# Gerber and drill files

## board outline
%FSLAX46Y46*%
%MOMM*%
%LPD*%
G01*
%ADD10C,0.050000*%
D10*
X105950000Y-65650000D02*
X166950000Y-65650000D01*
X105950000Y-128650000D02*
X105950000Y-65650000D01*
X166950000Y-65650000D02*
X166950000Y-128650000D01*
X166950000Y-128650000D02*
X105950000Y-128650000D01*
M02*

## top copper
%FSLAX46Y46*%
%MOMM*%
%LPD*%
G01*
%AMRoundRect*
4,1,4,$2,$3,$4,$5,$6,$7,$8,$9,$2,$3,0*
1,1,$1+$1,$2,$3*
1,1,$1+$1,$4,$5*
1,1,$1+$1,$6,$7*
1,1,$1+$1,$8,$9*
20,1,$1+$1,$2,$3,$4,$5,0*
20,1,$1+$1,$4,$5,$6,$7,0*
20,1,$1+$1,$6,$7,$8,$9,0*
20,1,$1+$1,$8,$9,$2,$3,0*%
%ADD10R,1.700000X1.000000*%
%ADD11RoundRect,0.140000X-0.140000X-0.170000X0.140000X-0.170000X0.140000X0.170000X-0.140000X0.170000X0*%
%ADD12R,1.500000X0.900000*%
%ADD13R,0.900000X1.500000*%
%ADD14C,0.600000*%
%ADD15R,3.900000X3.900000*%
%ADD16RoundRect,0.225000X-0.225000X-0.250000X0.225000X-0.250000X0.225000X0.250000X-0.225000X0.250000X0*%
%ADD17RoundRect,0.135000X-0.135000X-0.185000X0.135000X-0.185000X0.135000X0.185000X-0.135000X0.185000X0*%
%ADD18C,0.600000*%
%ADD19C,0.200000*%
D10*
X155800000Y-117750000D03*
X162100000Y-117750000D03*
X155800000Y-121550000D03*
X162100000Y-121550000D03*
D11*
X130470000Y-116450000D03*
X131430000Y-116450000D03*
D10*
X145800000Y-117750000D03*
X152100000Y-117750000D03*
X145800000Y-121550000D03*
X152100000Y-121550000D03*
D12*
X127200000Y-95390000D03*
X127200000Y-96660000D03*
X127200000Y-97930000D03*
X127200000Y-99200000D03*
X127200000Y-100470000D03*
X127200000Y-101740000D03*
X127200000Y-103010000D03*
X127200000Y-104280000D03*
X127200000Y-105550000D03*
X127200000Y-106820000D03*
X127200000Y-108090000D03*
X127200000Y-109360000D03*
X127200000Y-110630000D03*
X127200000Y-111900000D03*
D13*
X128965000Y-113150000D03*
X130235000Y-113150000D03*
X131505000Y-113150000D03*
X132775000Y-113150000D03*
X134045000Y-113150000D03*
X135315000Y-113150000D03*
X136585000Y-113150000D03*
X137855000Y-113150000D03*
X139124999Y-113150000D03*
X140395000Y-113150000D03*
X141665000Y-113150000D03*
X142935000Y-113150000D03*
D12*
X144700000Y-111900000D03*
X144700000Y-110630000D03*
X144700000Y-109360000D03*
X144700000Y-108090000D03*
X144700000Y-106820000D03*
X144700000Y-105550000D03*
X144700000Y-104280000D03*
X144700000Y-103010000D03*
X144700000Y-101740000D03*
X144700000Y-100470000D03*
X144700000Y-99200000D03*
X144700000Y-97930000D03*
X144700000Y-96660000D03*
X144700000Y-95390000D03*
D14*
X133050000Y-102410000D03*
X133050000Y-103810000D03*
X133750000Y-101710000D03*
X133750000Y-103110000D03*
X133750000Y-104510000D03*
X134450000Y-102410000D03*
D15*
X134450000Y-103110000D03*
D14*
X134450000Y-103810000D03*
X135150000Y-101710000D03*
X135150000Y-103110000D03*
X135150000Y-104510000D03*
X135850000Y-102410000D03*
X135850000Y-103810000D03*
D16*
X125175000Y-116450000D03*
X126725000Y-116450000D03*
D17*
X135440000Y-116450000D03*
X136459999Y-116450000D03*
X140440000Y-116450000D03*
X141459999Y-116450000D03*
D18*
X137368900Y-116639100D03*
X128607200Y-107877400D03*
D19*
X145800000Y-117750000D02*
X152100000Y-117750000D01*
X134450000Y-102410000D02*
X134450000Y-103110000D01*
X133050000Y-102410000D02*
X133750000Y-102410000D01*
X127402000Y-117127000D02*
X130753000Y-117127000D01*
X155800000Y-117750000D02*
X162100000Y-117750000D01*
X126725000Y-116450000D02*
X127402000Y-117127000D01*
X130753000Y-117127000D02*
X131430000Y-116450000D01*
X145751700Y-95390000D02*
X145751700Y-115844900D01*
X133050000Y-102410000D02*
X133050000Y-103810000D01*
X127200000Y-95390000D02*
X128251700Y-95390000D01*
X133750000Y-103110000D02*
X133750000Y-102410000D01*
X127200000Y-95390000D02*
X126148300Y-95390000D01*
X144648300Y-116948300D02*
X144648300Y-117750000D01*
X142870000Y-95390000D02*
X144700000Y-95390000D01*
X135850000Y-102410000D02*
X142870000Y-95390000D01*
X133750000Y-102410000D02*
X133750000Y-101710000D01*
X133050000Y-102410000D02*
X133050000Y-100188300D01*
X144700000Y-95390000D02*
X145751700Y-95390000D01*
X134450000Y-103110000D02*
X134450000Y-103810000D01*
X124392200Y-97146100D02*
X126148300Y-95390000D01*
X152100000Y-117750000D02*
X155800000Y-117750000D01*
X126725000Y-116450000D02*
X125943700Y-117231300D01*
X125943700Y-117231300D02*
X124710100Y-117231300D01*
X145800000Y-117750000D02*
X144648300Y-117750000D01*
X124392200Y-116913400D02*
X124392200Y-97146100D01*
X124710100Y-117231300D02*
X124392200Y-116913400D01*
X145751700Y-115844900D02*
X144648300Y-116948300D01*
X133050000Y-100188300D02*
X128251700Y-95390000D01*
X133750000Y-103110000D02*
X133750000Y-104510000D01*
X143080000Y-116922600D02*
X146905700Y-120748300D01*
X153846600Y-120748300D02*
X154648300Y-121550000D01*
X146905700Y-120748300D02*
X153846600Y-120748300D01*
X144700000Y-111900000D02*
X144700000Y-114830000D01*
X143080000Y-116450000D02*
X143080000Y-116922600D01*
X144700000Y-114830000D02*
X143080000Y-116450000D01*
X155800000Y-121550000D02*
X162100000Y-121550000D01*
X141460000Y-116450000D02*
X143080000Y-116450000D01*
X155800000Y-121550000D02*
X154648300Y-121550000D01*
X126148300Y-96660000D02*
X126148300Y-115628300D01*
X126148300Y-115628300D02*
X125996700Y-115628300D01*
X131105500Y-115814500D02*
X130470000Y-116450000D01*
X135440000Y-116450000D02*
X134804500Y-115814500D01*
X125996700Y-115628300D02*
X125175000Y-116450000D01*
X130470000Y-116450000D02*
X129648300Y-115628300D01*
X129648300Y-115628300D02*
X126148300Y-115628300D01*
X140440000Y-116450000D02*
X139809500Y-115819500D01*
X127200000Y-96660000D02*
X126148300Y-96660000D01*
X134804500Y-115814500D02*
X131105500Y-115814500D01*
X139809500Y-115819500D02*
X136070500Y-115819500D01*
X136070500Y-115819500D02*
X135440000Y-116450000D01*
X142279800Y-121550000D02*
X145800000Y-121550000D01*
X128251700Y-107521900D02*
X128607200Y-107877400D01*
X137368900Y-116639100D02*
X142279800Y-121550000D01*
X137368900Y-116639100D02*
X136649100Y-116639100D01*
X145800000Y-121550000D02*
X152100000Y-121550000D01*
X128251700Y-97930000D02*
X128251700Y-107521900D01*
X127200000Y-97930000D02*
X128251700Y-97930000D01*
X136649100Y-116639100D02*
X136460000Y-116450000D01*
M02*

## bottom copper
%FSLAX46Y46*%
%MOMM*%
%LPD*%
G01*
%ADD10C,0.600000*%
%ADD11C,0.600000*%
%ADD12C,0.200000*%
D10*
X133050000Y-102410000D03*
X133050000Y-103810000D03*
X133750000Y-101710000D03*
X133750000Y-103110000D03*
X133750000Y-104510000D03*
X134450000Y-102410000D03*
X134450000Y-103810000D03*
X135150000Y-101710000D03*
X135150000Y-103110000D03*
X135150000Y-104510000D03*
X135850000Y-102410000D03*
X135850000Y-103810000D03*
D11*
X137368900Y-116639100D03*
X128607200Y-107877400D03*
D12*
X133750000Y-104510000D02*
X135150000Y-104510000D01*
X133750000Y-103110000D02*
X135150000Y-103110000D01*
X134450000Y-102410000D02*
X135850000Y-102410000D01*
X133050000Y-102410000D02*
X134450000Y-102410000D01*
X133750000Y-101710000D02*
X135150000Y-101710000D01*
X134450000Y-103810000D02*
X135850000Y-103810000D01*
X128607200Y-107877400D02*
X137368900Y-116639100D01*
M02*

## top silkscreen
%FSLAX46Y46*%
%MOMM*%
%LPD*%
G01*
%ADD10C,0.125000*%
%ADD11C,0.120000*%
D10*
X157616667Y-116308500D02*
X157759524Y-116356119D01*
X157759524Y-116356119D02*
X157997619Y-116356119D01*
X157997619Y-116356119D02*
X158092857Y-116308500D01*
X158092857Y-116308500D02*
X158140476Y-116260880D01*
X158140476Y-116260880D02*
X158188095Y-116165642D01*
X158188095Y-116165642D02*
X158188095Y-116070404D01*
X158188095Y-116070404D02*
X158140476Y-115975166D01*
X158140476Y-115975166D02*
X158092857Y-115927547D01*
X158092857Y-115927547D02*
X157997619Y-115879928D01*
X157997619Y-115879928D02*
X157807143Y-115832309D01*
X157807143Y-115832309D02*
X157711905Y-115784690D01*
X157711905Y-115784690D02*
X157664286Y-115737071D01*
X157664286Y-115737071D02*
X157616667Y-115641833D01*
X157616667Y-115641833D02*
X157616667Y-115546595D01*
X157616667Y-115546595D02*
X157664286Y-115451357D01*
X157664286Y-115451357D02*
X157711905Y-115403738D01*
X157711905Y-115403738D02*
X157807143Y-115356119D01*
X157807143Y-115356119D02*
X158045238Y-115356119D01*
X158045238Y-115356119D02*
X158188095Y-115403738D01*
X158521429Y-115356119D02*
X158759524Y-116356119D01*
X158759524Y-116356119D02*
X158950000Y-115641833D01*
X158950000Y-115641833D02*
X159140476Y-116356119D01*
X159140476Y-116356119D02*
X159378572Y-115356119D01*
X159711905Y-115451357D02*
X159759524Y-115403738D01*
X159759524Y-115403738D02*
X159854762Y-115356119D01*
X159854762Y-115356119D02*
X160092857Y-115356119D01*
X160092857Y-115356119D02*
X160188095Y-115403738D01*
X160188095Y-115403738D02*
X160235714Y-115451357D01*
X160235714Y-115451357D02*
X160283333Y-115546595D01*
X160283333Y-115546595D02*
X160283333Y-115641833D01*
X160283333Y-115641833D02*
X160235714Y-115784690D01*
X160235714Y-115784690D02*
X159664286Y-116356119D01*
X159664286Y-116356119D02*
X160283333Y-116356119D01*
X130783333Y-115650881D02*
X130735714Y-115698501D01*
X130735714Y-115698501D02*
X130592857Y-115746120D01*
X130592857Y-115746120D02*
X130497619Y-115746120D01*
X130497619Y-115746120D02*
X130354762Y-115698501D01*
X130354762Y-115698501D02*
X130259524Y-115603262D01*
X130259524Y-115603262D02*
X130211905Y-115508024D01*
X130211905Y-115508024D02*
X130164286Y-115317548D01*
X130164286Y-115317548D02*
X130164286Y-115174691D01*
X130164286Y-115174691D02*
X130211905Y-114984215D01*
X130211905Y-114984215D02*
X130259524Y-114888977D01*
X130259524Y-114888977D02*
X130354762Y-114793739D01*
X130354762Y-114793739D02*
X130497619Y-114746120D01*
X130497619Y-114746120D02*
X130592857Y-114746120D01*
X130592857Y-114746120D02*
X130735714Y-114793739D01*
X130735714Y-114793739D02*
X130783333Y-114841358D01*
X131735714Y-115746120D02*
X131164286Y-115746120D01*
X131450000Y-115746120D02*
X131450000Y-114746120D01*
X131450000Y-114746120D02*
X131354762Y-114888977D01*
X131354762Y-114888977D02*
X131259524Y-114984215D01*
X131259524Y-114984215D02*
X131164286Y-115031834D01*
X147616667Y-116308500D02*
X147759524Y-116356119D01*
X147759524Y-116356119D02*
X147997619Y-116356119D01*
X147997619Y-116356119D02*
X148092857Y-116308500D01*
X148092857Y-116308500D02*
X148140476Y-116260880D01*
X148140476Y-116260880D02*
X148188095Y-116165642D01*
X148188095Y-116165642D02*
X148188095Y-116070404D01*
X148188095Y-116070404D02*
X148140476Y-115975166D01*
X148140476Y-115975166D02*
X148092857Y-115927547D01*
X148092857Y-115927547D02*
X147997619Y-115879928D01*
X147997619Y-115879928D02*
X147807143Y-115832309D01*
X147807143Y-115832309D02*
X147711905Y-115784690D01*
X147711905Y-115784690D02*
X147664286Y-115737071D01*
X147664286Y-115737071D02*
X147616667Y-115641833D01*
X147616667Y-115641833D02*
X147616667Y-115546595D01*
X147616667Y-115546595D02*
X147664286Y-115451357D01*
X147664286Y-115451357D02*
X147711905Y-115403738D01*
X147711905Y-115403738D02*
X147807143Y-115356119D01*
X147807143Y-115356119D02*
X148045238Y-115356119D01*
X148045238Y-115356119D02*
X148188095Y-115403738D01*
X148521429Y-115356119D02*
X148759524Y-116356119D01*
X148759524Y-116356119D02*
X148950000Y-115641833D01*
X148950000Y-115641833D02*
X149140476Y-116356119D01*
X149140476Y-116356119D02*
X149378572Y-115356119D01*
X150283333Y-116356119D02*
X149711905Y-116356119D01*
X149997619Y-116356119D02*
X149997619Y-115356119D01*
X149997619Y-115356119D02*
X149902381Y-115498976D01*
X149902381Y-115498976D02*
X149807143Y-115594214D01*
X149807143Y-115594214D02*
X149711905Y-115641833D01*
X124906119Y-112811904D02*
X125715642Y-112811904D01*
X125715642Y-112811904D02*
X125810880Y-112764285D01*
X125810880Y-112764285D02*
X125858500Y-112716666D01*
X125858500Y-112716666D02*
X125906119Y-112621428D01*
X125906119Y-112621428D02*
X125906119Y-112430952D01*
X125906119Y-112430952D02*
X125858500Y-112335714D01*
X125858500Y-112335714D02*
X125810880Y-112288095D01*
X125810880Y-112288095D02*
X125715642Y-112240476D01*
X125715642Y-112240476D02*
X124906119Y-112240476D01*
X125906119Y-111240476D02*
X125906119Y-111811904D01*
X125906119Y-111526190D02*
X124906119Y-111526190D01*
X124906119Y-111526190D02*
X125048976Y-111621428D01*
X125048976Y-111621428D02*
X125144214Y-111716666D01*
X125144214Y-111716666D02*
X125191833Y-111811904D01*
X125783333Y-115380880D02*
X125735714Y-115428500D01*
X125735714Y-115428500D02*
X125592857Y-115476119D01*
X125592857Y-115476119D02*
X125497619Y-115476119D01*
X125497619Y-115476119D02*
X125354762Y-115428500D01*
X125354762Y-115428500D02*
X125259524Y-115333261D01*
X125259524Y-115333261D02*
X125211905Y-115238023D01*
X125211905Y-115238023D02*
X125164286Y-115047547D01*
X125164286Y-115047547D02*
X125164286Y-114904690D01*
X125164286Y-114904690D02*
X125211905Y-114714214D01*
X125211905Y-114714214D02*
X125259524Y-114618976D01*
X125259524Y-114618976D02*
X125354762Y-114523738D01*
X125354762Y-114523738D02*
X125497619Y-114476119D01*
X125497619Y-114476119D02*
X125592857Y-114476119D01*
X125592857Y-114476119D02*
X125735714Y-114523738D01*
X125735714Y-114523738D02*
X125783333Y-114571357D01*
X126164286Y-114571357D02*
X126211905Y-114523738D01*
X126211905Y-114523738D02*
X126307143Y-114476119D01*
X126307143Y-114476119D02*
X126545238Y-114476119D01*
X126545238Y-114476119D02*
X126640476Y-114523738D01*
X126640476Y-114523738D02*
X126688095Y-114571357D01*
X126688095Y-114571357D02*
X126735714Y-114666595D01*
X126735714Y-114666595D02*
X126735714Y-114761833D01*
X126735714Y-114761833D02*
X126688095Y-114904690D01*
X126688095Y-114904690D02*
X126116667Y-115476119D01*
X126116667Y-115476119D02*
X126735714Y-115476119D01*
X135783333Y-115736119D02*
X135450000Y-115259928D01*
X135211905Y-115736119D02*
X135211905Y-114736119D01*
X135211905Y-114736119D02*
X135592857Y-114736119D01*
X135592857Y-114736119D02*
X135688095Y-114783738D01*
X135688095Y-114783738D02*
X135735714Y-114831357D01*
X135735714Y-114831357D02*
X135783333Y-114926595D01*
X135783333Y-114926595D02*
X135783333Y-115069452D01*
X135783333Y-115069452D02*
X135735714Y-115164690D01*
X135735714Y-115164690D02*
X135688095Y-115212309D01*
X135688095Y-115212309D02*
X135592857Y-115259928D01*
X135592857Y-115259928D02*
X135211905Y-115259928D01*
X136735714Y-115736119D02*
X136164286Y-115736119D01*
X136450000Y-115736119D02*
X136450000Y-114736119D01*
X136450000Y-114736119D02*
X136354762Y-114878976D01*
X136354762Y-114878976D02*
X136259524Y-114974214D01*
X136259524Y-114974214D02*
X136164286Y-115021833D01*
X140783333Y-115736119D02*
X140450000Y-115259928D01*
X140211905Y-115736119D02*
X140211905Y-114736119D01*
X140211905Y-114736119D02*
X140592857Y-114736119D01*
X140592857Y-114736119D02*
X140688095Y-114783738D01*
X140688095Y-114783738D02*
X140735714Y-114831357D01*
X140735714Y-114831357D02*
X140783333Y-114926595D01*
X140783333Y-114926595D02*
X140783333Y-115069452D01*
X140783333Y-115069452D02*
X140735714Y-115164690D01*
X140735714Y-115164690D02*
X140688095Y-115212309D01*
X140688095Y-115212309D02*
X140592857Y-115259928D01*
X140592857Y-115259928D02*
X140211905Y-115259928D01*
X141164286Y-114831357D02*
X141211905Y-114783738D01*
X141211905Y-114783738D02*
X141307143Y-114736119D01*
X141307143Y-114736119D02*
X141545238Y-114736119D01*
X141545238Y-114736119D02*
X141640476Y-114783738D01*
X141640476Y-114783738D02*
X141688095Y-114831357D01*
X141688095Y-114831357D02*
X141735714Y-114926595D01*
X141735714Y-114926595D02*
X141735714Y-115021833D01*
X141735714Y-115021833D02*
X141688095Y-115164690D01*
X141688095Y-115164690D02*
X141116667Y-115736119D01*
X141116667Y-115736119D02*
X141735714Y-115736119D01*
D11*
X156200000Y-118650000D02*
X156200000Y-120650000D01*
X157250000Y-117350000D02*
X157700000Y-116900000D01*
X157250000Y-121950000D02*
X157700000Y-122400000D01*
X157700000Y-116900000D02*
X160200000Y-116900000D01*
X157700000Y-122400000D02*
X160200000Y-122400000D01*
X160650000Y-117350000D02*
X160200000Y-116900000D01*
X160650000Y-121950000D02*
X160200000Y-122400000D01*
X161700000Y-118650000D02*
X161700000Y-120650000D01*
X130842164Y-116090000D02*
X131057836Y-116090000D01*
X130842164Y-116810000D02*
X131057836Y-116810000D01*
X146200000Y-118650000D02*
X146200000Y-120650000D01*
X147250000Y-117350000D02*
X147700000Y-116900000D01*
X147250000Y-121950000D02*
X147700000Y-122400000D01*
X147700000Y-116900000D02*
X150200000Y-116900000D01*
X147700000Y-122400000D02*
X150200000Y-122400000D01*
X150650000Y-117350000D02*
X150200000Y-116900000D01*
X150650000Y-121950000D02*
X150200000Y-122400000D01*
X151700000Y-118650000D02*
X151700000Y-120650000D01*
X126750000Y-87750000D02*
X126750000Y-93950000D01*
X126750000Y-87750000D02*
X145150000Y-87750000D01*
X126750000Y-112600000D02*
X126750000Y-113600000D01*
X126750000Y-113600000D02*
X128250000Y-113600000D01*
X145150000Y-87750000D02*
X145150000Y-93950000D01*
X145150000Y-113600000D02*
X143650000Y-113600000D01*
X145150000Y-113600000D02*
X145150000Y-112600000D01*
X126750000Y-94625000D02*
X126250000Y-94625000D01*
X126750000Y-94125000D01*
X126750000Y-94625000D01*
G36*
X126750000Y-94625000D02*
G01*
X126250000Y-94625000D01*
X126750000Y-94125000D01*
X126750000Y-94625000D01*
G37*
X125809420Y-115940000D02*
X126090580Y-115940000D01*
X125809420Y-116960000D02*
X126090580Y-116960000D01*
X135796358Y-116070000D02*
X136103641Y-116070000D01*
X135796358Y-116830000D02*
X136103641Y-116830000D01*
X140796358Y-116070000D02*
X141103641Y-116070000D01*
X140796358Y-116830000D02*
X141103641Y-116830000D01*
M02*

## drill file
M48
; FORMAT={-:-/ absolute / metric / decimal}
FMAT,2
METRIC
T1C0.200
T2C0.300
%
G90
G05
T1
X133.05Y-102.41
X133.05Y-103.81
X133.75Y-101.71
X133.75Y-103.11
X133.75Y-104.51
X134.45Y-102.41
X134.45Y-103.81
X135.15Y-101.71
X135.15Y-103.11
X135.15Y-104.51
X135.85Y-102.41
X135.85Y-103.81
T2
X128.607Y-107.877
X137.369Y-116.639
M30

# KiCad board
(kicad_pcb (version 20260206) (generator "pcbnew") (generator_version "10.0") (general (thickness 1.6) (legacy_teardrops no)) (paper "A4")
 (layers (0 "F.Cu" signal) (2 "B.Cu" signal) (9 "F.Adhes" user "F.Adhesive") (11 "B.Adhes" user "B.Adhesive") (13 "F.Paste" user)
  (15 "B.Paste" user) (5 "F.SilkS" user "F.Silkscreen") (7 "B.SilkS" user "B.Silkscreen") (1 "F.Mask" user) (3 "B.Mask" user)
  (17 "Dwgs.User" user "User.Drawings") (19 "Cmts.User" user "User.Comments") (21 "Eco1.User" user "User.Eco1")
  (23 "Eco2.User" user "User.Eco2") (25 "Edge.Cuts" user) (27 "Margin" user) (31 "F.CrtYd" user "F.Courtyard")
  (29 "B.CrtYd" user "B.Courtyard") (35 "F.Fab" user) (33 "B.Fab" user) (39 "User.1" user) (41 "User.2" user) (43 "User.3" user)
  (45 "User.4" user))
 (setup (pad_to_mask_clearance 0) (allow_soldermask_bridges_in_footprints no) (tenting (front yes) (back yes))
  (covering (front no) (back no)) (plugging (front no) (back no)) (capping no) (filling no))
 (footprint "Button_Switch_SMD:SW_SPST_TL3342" (layer "F.Cu") (at 158.95 119.65)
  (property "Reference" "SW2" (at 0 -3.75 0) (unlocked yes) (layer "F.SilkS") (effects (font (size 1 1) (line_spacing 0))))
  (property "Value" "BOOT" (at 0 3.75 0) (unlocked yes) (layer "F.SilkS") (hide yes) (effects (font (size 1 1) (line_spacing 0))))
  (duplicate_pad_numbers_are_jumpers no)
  (fp_line (start -2.75 -1) (end -2.75 1) (stroke (width 0.12) (type solid)) (layer "F.SilkS"))
  (fp_line (start -1.7 -2.3) (end -1.25 -2.75) (stroke (width 0.12) (type solid)) (layer "F.SilkS"))
  (fp_line (start -1.7 2.3) (end -1.25 2.75) (stroke (width 0.12) (type solid)) (layer "F.SilkS"))
  (fp_line (start -1.25 -2.75) (end 1.25 -2.75) (stroke (width 0.12) (type solid)) (layer "F.SilkS"))
  (fp_line (start -1.25 2.75) (end 1.25 2.75) (stroke (width 0.12) (type solid)) (layer "F.SilkS"))
  (fp_line (start 1.7 -2.3) (end 1.25 -2.75) (stroke (width 0.12) (type solid)) (layer "F.SilkS"))
  (fp_line (start 1.7 2.3) (end 1.25 2.75) (stroke (width 0.12) (type solid)) (layer "F.SilkS"))
  (fp_line (start 2.75 -1) (end 2.75 1) (stroke (width 0.12) (type solid)) (layer "F.SilkS"))
  (pad "1" smd rect (at -3.15 -1.9) (size 1.7 1) (layers "F.Cu" "F.Mask" "F.Paste") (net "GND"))
  (pad "1" smd rect (at 3.15 -1.9) (size 1.7 1) (layers "F.Cu" "F.Mask" "F.Paste") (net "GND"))
  (pad "2" smd rect (at -3.15 1.9) (size 1.7 1) (layers "F.Cu" "F.Mask" "F.Paste") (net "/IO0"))
  (pad "2" smd rect (at 3.15 1.9) (size 1.7 1) (layers "F.Cu" "F.Mask" "F.Paste") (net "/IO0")))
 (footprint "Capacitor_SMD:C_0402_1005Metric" (layer "F.Cu") (at 130.95 116.45)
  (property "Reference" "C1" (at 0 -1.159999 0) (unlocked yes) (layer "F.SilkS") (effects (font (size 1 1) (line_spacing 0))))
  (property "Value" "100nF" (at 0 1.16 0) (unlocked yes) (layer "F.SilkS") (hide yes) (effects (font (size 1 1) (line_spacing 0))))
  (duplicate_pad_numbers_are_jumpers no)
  (fp_line (start -0.107836 -0.36) (end 0.107836 -0.36) (stroke (width 0.12) (type solid)) (layer "F.SilkS"))
  (fp_line (start -0.107836 0.36) (end 0.107836 0.36) (stroke (width 0.12) (type solid)) (layer "F.SilkS"))
  (pad "1" smd roundrect (at -0.48 0) (size 0.56 0.62) (layers "F.Cu" "F.Mask" "F.Paste") (roundrect_rratio 0.25) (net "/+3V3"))
  (pad "2" smd roundrect (at 0.48 0) (size 0.56 0.62) (layers "F.Cu" "F.Mask" "F.Paste") (roundrect_rratio 0.25) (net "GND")))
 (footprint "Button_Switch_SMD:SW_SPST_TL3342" (layer "F.Cu") (at 148.95 119.65)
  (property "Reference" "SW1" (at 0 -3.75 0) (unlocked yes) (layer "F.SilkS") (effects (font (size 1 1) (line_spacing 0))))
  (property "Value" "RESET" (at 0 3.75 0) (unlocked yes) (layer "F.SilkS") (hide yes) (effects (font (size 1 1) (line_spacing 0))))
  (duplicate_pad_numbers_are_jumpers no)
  (fp_line (start -2.75 -1) (end -2.75 1) (stroke (width 0.12) (type solid)) (layer "F.SilkS"))
  (fp_line (start -1.7 -2.3) (end -1.25 -2.75) (stroke (width 0.12) (type solid)) (layer "F.SilkS"))
  (fp_line (start -1.7 2.3) (end -1.25 2.75) (stroke (width 0.12) (type solid)) (layer "F.SilkS"))
  (fp_line (start -1.25 -2.75) (end 1.25 -2.75) (stroke (width 0.12) (type solid)) (layer "F.SilkS"))
  (fp_line (start -1.25 2.75) (end 1.25 2.75) (stroke (width 0.12) (type solid)) (layer "F.SilkS"))
  (fp_line (start 1.7 -2.3) (end 1.25 -2.75) (stroke (width 0.12) (type solid)) (layer "F.SilkS"))
  (fp_line (start 1.7 2.3) (end 1.25 2.75) (stroke (width 0.12) (type solid)) (layer "F.SilkS"))
  (fp_line (start 2.75 -1) (end 2.75 1) (stroke (width 0.12) (type solid)) (layer "F.SilkS"))
  (pad "1" smd rect (at -3.15 -1.9) (size 1.7 1) (layers "F.Cu" "F.Mask" "F.Paste") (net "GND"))
  (pad "1" smd rect (at 3.15 -1.9) (size 1.7 1) (layers "F.Cu" "F.Mask" "F.Paste") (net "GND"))
  (pad "2" smd rect (at -3.15 1.9) (size 1.7 1) (layers "F.Cu" "F.Mask" "F.Paste") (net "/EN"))
  (pad "2" smd rect (at 3.15 1.9) (size 1.7 1) (layers "F.Cu" "F.Mask" "F.Paste") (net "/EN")))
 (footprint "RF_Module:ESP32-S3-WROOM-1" (layer "F.Cu") (at 135.95 100.65)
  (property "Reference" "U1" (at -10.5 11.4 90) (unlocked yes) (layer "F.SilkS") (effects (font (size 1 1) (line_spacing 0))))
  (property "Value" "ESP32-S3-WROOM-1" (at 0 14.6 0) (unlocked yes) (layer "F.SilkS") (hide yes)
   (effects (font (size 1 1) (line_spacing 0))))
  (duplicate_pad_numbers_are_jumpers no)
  (fp_line (start -9.2 -12.9) (end -9.2 -6.7) (stroke (width 0.12) (type solid)) (layer "F.SilkS"))
  (fp_line (start -9.2 -12.9) (end 9.2 -12.9) (stroke (width 0.12) (type solid)) (layer "F.SilkS"))
  (fp_line (start -9.2 11.95) (end -9.2 12.95) (stroke (width 0.12) (type solid)) (layer "F.SilkS"))
  (fp_line (start -9.2 12.95) (end -7.7 12.95) (stroke (width 0.12) (type solid)) (layer "F.SilkS"))
  (fp_line (start 9.2 -12.9) (end 9.2 -6.7) (stroke (width 0.12) (type solid)) (layer "F.SilkS"))
  (fp_line (start 9.2 12.95) (end 7.7 12.95) (stroke (width 0.12) (type solid)) (layer "F.SilkS"))
  (fp_line (start 9.2 12.95) (end 9.2 11.95) (stroke (width 0.12) (type solid)) (layer "F.SilkS"))
  (fp_poly
   (pts (xy -9.2 -6.025) (xy -9.7 -6.025) (xy -9.2 -6.525) (xy -9.2 -6.025)) (stroke (width 0.12) (type solid)) (fill yes) (layer "F.SilkS"))
  (pad "" smd rect (at -2.9 1.06) (size 0.9 0.9) (layers "F.Paste"))
  (pad "" smd rect (at -2.9 2.46 270) (size 0.9 0.9) (layers "F.Paste"))
  (pad "" smd rect (at -2.9 3.86) (size 0.9 0.9) (layers "F.Paste"))
  (pad "" smd rect (at -1.5 1.06 270) (size 0.9 0.9) (layers "F.Paste"))
  (pad "" smd rect (at -1.5 2.46 270) (size 0.9 0.9) (layers "F.Paste"))
  (pad "" smd rect (at -1.5 3.86 270) (size 0.9 0.9) (layers "F.Paste"))
  (pad "" smd rect (at -0.1 1.06 270) (size 0.9 0.9) (layers "F.Paste"))
  (pad "" smd rect (at -0.1 2.46 270) (size 0.9 0.9) (layers "F.Paste"))
  (pad "" smd rect (at -0.1 3.86 270) (size 0.9 0.9) (layers "F.Paste"))
  (pad "1" smd rect (at -8.75 -5.26) (size 1.5 0.9) (layers "F.Cu" "F.Mask" "F.Paste") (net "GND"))
  (pad "2" smd rect (at -8.75 -3.99) (size 1.5 0.9) (layers "F.Cu" "F.Mask" "F.Paste") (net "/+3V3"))
  (pad "3" smd rect (at -8.75 -2.72) (size 1.5 0.9) (layers "F.Cu" "F.Mask" "F.Paste") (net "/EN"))
  (pad "4" smd rect (at -8.75 -1.45) (size 1.5 0.9) (layers "F.Cu" "F.Mask" "F.Paste") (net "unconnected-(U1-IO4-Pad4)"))
  (pad "5" smd rect (at -8.75 -0.18) (size 1.5 0.9) (layers "F.Cu" "F.Mask" "F.Paste") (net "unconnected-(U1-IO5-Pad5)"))
  (pad "6" smd rect (at -8.75 1.09) (size 1.5 0.9) (layers "F.Cu" "F.Mask" "F.Paste") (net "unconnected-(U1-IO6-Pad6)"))
  (pad "7" smd rect (at -8.75 2.36) (size 1.5 0.9) (layers "F.Cu" "F.Mask" "F.Paste") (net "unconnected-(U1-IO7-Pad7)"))
  (pad "8" smd rect (at -8.75 3.63) (size 1.5 0.9) (layers "F.Cu" "F.Mask" "F.Paste") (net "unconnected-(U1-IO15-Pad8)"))
  (pad "9" smd rect (at -8.75 4.9) (size 1.5 0.9) (layers "F.Cu" "F.Mask" "F.Paste") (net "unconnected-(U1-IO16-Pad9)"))
  (pad "10" smd rect (at -8.75 6.17) (size 1.5 0.9) (layers "F.Cu" "F.Mask" "F.Paste") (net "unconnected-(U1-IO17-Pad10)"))
  (pad "11" smd rect (at -8.75 7.44) (size 1.5 0.9) (layers "F.Cu" "F.Mask" "F.Paste") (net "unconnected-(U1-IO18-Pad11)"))
  (pad "12" smd rect (at -8.75 8.71) (size 1.5 0.9) (layers "F.Cu" "F.Mask" "F.Paste") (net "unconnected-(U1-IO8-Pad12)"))
  (pad "13" smd rect (at -8.75 9.98) (size 1.5 0.9) (layers "F.Cu" "F.Mask" "F.Paste") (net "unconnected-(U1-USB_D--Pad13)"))
  (pad "14" smd rect (at -8.75 11.25 180) (size 1.5 0.9) (layers "F.Cu" "F.Mask" "F.Paste") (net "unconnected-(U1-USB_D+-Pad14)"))
  (pad "15" smd rect (at -6.985 12.5 270) (size 1.5 0.9) (layers "F.Cu" "F.Mask" "F.Paste") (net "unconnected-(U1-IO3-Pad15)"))
  (pad "16" smd rect (at -5.715 12.5 270) (size 1.5 0.9) (layers "F.Cu" "F.Mask" "F.Paste") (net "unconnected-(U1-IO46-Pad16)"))
  (pad "17" smd rect (at -4.445 12.5 270) (size 1.5 0.9) (layers "F.Cu" "F.Mask" "F.Paste") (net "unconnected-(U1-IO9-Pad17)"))
  (pad "18" smd rect (at -3.175 12.5 270) (size 1.5 0.9) (layers "F.Cu" "F.Mask" "F.Paste") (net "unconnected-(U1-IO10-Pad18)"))
  (pad "19" smd rect (at -1.905 12.5 270) (size 1.5 0.9) (layers "F.Cu" "F.Mask" "F.Paste") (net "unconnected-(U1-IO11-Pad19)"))
  (pad "20" smd rect (at -0.635 12.5 270) (size 1.5 0.9) (layers "F.Cu" "F.Mask" "F.Paste") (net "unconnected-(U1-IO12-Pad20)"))
  (pad "21" smd rect (at 0.635 12.5 270) (size 1.5 0.9) (layers "F.Cu" "F.Mask" "F.Paste") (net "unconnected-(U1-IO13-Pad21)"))
  (pad "22" smd rect (at 1.905 12.5 270) (size 1.5 0.9) (layers "F.Cu" "F.Mask" "F.Paste") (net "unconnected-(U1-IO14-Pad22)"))
  (pad "23" smd rect (at 3.174999 12.5 270) (size 1.5 0.9) (layers "F.Cu" "F.Mask" "F.Paste") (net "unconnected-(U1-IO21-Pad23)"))
  (pad "24" smd rect (at 4.445 12.5 270) (size 1.5 0.9) (layers "F.Cu" "F.Mask" "F.Paste") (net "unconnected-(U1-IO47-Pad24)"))
  (pad "25" smd rect (at 5.715 12.5 270) (size 1.5 0.9) (layers "F.Cu" "F.Mask" "F.Paste") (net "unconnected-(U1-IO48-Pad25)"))
  (pad "26" smd rect (at 6.985 12.5 270) (size 1.5 0.9) (layers "F.Cu" "F.Mask" "F.Paste") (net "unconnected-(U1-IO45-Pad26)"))
  (pad "27" smd rect (at 8.75 11.25) (size 1.5 0.9) (layers "F.Cu" "F.Mask" "F.Paste") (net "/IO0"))
  (pad "28" smd rect (at 8.75 9.98) (size 1.5 0.9) (layers "F.Cu" "F.Mask" "F.Paste") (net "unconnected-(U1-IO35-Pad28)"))
  (pad "29" smd rect (at 8.75 8.71) (size 1.5 0.9) (layers "F.Cu" "F.Mask" "F.Paste") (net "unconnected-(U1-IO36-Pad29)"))
  (pad "30" smd rect (at 8.75 7.44) (size 1.5 0.9) (layers "F.Cu" "F.Mask" "F.Paste") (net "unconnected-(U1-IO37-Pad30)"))
  (pad "31" smd rect (at 8.75 6.17) (size 1.5 0.9) (layers "F.Cu" "F.Mask" "F.Paste") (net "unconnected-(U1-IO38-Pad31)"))
  (pad "32" smd rect (at 8.75 4.9) (size 1.5 0.9) (layers "F.Cu" "F.Mask" "F.Paste") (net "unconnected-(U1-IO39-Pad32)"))
  (pad "33" smd rect (at 8.75 3.63) (size 1.5 0.9) (layers "F.Cu" "F.Mask" "F.Paste") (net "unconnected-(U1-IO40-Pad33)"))
  (pad "34" smd rect (at 8.75 2.36) (size 1.5 0.9) (layers "F.Cu" "F.Mask" "F.Paste") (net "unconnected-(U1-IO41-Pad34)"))
  (pad "35" smd rect (at 8.75 1.09) (size 1.5 0.9) (layers "F.Cu" "F.Mask" "F.Paste") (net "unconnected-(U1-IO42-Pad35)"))
  (pad "36" smd rect (at 8.75 -0.18) (size 1.5 0.9) (layers "F.Cu" "F.Mask" "F.Paste") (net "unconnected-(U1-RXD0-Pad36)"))
  (pad "37" smd rect (at 8.75 -1.45) (size 1.5 0.9) (layers "F.Cu" "F.Mask" "F.Paste") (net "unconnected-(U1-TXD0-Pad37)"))
  (pad "38" smd rect (at 8.75 -2.72) (size 1.5 0.9) (layers "F.Cu" "F.Mask" "F.Paste") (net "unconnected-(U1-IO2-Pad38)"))
  (pad "39" smd rect (at 8.75 -3.99) (size 1.5 0.9) (layers "F.Cu" "F.Mask" "F.Paste") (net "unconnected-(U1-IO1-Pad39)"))
  (pad "40" smd rect (at 8.75 -5.26) (size 1.5 0.9) (layers "F.Cu" "F.Mask" "F.Paste") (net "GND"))
  (pad "41" thru_hole circle (at -2.9 1.76 90) (size 0.6 0.6) (drill 0.2) (layers "*.Cu" "F.Mask") (remove_unused_layers no) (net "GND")
   (zone_connect 2))
  (pad "41" thru_hole circle (at -2.9 3.16) (size 0.6 0.6) (drill 0.2) (layers "*.Cu" "F.Mask") (remove_unused_layers no) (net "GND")
   (zone_connect 2))
  (pad "41" thru_hole circle (at -2.2 1.06) (size 0.6 0.6) (drill 0.2) (layers "*.Cu" "F.Mask") (remove_unused_layers no) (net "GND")
   (zone_connect 2))
  (pad "41" thru_hole circle (at -2.2 2.46) (size 0.6 0.6) (drill 0.2) (layers "*.Cu" "F.Mask") (remove_unused_layers no) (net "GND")
   (zone_connect 2))
  (pad "41" thru_hole circle (at -2.2 3.86) (size 0.6 0.6) (drill 0.2) (layers "*.Cu" "F.Mask") (remove_unused_layers no) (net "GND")
   (zone_connect 2))
  (pad "41" thru_hole circle (at -1.5 1.76) (size 0.6 0.6) (drill 0.2) (layers "*.Cu" "F.Mask") (remove_unused_layers no) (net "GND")
   (zone_connect 2))
  (pad "41" smd rect (at -1.5 2.46 270) (size 3.9 3.9) (layers "F.Cu" "F.Mask") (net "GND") (zone_connect 2))
  (pad "41" thru_hole circle (at -1.5 3.16) (size 0.6 0.6) (drill 0.2) (layers "*.Cu" "F.Mask") (remove_unused_layers no) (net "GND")
   (zone_connect 2))
  (pad "41" thru_hole circle (at -0.8 1.06) (size 0.6 0.6) (drill 0.2) (layers "*.Cu" "F.Mask") (remove_unused_layers no) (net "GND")
   (zone_connect 2))
  (pad "41" thru_hole circle (at -0.8 2.46) (size 0.6 0.6) (drill 0.2) (layers "*.Cu" "F.Mask") (remove_unused_layers no) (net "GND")
   (zone_connect 2))
  (pad "41" thru_hole circle (at -0.8 3.86) (size 0.6 0.6) (drill 0.2) (layers "*.Cu" "F.Mask") (remove_unused_layers no) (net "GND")
   (zone_connect 2))
  (pad "41" thru_hole circle (at -0.1 1.76) (size 0.6 0.6) (drill 0.2) (layers "*.Cu" "F.Mask") (remove_unused_layers no) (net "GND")
   (zone_connect 2))
  (pad "41" thru_hole circle (at -0.1 3.16) (size 0.6 0.6) (drill 0.2) (layers "*.Cu" "F.Mask") (remove_unused_layers no) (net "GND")
   (zone_connect 2))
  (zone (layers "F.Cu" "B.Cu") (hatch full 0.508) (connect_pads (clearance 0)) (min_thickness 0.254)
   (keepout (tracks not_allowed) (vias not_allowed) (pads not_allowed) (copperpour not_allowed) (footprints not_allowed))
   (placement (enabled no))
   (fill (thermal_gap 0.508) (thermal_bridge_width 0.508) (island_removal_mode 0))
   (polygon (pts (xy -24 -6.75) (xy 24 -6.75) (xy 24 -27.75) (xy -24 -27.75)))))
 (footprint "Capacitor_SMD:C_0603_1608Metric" (layer "F.Cu") (at 125.95 116.45)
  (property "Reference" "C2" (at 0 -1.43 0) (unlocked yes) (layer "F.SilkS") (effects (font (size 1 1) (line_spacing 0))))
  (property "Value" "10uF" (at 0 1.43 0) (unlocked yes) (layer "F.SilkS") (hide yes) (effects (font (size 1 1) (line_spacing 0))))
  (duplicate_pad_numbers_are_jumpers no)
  (fp_line (start -0.14058 -0.51) (end 0.14058 -0.51) (stroke (width 0.12) (type solid)) (layer "F.SilkS"))
  (fp_line (start -0.14058 0.51) (end 0.14058 0.51) (stroke (width 0.12) (type solid)) (layer "F.SilkS"))
  (pad "1" smd roundrect (at -0.775 0) (size 0.9 0.95) (layers "F.Cu" "F.Mask" "F.Paste") (roundrect_rratio 0.25) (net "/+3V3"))
  (pad "2" smd roundrect (at 0.775 0) (size 0.9 0.95) (layers "F.Cu" "F.Mask" "F.Paste") (roundrect_rratio 0.25) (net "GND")))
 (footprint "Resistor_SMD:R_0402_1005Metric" (layer "F.Cu") (at 135.95 116.45)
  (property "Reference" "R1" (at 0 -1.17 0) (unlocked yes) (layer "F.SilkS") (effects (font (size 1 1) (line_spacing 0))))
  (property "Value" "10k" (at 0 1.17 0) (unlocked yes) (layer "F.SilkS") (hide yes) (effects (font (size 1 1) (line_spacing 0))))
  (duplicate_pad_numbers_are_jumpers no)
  (fp_line (start -0.153642 -0.38) (end 0.153641 -0.38) (stroke (width 0.12) (type solid)) (layer "F.SilkS"))
  (fp_line (start -0.153642 0.38) (end 0.153641 0.38) (stroke (width 0.12) (type solid)) (layer "F.SilkS"))
  (pad "1" smd roundrect (at -0.51 0) (size 0.54 0.64) (layers "F.Cu" "F.Mask" "F.Paste") (roundrect_rratio 0.25) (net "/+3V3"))
  (pad "2" smd roundrect (at 0.509999 0) (size 0.54 0.64) (layers "F.Cu" "F.Mask" "F.Paste") (roundrect_rratio 0.25) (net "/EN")))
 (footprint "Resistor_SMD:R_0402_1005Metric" (layer "F.Cu") (at 140.95 116.45)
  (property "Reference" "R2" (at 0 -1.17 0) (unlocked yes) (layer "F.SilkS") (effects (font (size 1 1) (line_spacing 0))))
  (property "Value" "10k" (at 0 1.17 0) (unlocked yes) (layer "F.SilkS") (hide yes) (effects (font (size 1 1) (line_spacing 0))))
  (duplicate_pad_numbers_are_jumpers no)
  (fp_line (start -0.153642 -0.38) (end 0.153641 -0.38) (stroke (width 0.12) (type solid)) (layer "F.SilkS"))
  (fp_line (start -0.153642 0.38) (end 0.153641 0.38) (stroke (width 0.12) (type solid)) (layer "F.SilkS"))
  (pad "1" smd roundrect (at -0.51 0) (size 0.54 0.64) (layers "F.Cu" "F.Mask" "F.Paste") (roundrect_rratio 0.25) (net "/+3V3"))
  (pad "2" smd roundrect (at 0.509999 0) (size 0.54 0.64) (layers "F.Cu" "F.Mask" "F.Paste") (roundrect_rratio 0.25) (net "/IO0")))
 (gr_line (start 105.95 65.65) (end 166.95 65.65) (stroke (width 0.05) (type default)) (layer "Edge.Cuts"))
 (gr_line (start 105.95 128.65) (end 105.95 65.65) (stroke (width 0.05) (type default)) (layer "Edge.Cuts"))
 (gr_line (start 166.95 65.65) (end 166.95 128.65) (stroke (width 0.05) (type default)) (layer "Edge.Cuts"))
 (gr_line (start 166.95 128.65) (end 105.95 128.65) (stroke (width 0.05) (type default)) (layer "Edge.Cuts"))
 (segment (start 145.8 117.75) (end 152.1 117.75) (width 0.2) (layer "F.Cu") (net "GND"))
 (segment (start 134.45 102.41) (end 134.45 103.11) (width 0.2) (layer "F.Cu") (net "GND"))
 (segment (start 133.05 102.41) (end 133.75 102.41) (width 0.2) (layer "F.Cu") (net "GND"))
 (segment (start 127.402 117.127) (end 130.753 117.127) (width 0.2) (layer "F.Cu") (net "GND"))
 (segment (start 155.8 117.75) (end 162.1 117.75) (width 0.2) (layer "F.Cu") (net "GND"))
 (segment (start 126.725 116.45) (end 127.402 117.127) (width 0.2) (layer "F.Cu") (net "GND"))
 (segment (start 130.753 117.127) (end 131.43 116.45) (width 0.2) (layer "F.Cu") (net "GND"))
 (segment (start 145.7517 95.39) (end 145.7517 115.8449) (width 0.2) (layer "F.Cu") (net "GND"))
 (segment (start 133.05 102.41) (end 133.05 103.81) (width 0.2) (layer "F.Cu") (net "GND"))
 (segment (start 127.2 95.39) (end 128.2517 95.39) (width 0.2) (layer "F.Cu") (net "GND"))
 (segment (start 133.75 103.11) (end 133.75 102.41) (width 0.2) (layer "F.Cu") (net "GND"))
 (segment (start 127.2 95.39) (end 126.1483 95.39) (width 0.2) (layer "F.Cu") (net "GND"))
 (segment (start 144.6483 116.9483) (end 144.6483 117.75) (width 0.2) (layer "F.Cu") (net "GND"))
 (segment (start 142.87 95.39) (end 144.7 95.39) (width 0.2) (layer "F.Cu") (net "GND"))
 (segment (start 135.85 102.41) (end 142.87 95.39) (width 0.2) (layer "F.Cu") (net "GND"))
 (segment (start 133.75 102.41) (end 133.75 101.71) (width 0.2) (layer "F.Cu") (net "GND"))
 (segment (start 133.05 102.41) (end 133.05 100.1883) (width 0.2) (layer "F.Cu") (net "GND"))
 (segment (start 144.7 95.39) (end 145.7517 95.39) (width 0.2) (layer "F.Cu") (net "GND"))
 (segment (start 134.45 103.11) (end 134.45 103.81) (width 0.2) (layer "F.Cu") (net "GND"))
 (segment (start 124.3922 97.1461) (end 126.1483 95.39) (width 0.2) (layer "F.Cu") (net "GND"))
 (segment (start 152.1 117.75) (end 155.8 117.75) (width 0.2) (layer "F.Cu") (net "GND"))
 (segment (start 126.725 116.45) (end 125.9437 117.2313) (width 0.2) (layer "F.Cu") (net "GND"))
 (segment (start 125.9437 117.2313) (end 124.7101 117.2313) (width 0.2) (layer "F.Cu") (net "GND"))
 (segment (start 145.8 117.75) (end 144.6483 117.75) (width 0.2) (layer "F.Cu") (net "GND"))
 (segment (start 124.3922 116.9134) (end 124.3922 97.1461) (width 0.2) (layer "F.Cu") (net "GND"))
 (segment (start 124.7101 117.2313) (end 124.3922 116.9134) (width 0.2) (layer "F.Cu") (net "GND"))
 (segment (start 145.7517 115.8449) (end 144.6483 116.9483) (width 0.2) (layer "F.Cu") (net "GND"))
 (segment (start 133.05 100.1883) (end 128.2517 95.39) (width 0.2) (layer "F.Cu") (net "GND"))
 (segment (start 133.75 103.11) (end 133.75 104.51) (width 0.2) (layer "F.Cu") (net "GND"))
 (segment (start 133.75 104.51) (end 135.15 104.51) (width 0.2) (layer "B.Cu") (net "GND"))
 (segment (start 133.75 103.11) (end 135.15 103.11) (width 0.2) (layer "B.Cu") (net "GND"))
 (segment (start 134.45 102.41) (end 135.85 102.41) (width 0.2) (layer "B.Cu") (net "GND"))
 (segment (start 133.05 102.41) (end 134.45 102.41) (width 0.2) (layer "B.Cu") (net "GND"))
 (segment (start 133.75 101.71) (end 135.15 101.71) (width 0.2) (layer "B.Cu") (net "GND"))
 (segment (start 134.45 103.81) (end 135.85 103.81) (width 0.2) (layer "B.Cu") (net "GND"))
 (segment (start 143.08 116.9226) (end 146.9057 120.7483) (width 0.2) (layer "F.Cu") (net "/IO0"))
 (segment (start 153.8466 120.7483) (end 154.6483 121.55) (width 0.2) (layer "F.Cu") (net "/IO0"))
 (segment (start 146.9057 120.7483) (end 153.8466 120.7483) (width 0.2) (layer "F.Cu") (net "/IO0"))
 (segment (start 144.7 111.9) (end 144.7 114.83) (width 0.2) (layer "F.Cu") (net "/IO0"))
 (segment (start 143.08 116.45) (end 143.08 116.9226) (width 0.2) (layer "F.Cu") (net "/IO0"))
 (segment (start 144.7 114.83) (end 143.08 116.45) (width 0.2) (layer "F.Cu") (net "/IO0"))
 (segment (start 155.8 121.55) (end 162.1 121.55) (width 0.2) (layer "F.Cu") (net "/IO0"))
 (segment (start 141.46 116.45) (end 143.08 116.45) (width 0.2) (layer "F.Cu") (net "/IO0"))
 (segment (start 155.8 121.55) (end 154.6483 121.55) (width 0.2) (layer "F.Cu") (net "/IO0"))
 (segment (start 126.1483 96.66) (end 126.1483 115.6283) (width 0.2) (layer "F.Cu") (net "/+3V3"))
 (segment (start 126.1483 115.6283) (end 125.9967 115.6283) (width 0.2) (layer "F.Cu") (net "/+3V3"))
 (segment (start 131.1055 115.8145) (end 130.47 116.45) (width 0.2) (layer "F.Cu") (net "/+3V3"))
 (segment (start 135.44 116.45) (end 134.8045 115.8145) (width 0.2) (layer "F.Cu") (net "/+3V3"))
 (segment (start 125.9967 115.6283) (end 125.175 116.45) (width 0.2) (layer "F.Cu") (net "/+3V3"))
 (segment (start 130.47 116.45) (end 129.6483 115.6283) (width 0.2) (layer "F.Cu") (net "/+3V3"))
 (segment (start 129.6483 115.6283) (end 126.1483 115.6283) (width 0.2) (layer "F.Cu") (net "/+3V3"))
 (segment (start 140.44 116.45) (end 139.8095 115.8195) (width 0.2) (layer "F.Cu") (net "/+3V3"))
 (segment (start 127.2 96.66) (end 126.1483 96.66) (width 0.2) (layer "F.Cu") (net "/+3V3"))
 (segment (start 134.8045 115.8145) (end 131.1055 115.8145) (width 0.2) (layer "F.Cu") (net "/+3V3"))
 (segment (start 139.8095 115.8195) (end 136.0705 115.8195) (width 0.2) (layer "F.Cu") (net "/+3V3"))
 (segment (start 136.0705 115.8195) (end 135.44 116.45) (width 0.2) (layer "F.Cu") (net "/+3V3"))
 (segment (start 142.2798 121.55) (end 145.8 121.55) (width 0.2) (layer "F.Cu") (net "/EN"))
 (segment (start 128.2517 107.5219) (end 128.6072 107.8774) (width 0.2) (layer "F.Cu") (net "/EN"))
 (segment (start 137.3689 116.6391) (end 142.2798 121.55) (width 0.2) (layer "F.Cu") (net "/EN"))
 (segment (start 137.3689 116.6391) (end 136.6491 116.6391) (width 0.2) (layer "F.Cu") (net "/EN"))
 (segment (start 145.8 121.55) (end 152.1 121.55) (width 0.2) (layer "F.Cu") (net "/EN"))
 (segment (start 128.2517 97.93) (end 128.2517 107.5219) (width 0.2) (layer "F.Cu") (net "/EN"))
 (segment (start 127.2 97.93) (end 128.2517 97.93) (width 0.2) (layer "F.Cu") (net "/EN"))
 (segment (start 136.6491 116.6391) (end 136.46 116.45) (width 0.2) (layer "F.Cu") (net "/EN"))
 (via (at 137.3689 116.6391) (size 0.6) (drill 0.3) (layers "F.Cu" "B.Cu") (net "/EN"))
 (via (at 128.6072 107.8774) (size 0.6) (drill 0.3) (layers "F.Cu" "B.Cu") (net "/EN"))
 (segment (start 128.6072 107.8774) (end 137.3689 116.6391) (width 0.2) (layer "B.Cu") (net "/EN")))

